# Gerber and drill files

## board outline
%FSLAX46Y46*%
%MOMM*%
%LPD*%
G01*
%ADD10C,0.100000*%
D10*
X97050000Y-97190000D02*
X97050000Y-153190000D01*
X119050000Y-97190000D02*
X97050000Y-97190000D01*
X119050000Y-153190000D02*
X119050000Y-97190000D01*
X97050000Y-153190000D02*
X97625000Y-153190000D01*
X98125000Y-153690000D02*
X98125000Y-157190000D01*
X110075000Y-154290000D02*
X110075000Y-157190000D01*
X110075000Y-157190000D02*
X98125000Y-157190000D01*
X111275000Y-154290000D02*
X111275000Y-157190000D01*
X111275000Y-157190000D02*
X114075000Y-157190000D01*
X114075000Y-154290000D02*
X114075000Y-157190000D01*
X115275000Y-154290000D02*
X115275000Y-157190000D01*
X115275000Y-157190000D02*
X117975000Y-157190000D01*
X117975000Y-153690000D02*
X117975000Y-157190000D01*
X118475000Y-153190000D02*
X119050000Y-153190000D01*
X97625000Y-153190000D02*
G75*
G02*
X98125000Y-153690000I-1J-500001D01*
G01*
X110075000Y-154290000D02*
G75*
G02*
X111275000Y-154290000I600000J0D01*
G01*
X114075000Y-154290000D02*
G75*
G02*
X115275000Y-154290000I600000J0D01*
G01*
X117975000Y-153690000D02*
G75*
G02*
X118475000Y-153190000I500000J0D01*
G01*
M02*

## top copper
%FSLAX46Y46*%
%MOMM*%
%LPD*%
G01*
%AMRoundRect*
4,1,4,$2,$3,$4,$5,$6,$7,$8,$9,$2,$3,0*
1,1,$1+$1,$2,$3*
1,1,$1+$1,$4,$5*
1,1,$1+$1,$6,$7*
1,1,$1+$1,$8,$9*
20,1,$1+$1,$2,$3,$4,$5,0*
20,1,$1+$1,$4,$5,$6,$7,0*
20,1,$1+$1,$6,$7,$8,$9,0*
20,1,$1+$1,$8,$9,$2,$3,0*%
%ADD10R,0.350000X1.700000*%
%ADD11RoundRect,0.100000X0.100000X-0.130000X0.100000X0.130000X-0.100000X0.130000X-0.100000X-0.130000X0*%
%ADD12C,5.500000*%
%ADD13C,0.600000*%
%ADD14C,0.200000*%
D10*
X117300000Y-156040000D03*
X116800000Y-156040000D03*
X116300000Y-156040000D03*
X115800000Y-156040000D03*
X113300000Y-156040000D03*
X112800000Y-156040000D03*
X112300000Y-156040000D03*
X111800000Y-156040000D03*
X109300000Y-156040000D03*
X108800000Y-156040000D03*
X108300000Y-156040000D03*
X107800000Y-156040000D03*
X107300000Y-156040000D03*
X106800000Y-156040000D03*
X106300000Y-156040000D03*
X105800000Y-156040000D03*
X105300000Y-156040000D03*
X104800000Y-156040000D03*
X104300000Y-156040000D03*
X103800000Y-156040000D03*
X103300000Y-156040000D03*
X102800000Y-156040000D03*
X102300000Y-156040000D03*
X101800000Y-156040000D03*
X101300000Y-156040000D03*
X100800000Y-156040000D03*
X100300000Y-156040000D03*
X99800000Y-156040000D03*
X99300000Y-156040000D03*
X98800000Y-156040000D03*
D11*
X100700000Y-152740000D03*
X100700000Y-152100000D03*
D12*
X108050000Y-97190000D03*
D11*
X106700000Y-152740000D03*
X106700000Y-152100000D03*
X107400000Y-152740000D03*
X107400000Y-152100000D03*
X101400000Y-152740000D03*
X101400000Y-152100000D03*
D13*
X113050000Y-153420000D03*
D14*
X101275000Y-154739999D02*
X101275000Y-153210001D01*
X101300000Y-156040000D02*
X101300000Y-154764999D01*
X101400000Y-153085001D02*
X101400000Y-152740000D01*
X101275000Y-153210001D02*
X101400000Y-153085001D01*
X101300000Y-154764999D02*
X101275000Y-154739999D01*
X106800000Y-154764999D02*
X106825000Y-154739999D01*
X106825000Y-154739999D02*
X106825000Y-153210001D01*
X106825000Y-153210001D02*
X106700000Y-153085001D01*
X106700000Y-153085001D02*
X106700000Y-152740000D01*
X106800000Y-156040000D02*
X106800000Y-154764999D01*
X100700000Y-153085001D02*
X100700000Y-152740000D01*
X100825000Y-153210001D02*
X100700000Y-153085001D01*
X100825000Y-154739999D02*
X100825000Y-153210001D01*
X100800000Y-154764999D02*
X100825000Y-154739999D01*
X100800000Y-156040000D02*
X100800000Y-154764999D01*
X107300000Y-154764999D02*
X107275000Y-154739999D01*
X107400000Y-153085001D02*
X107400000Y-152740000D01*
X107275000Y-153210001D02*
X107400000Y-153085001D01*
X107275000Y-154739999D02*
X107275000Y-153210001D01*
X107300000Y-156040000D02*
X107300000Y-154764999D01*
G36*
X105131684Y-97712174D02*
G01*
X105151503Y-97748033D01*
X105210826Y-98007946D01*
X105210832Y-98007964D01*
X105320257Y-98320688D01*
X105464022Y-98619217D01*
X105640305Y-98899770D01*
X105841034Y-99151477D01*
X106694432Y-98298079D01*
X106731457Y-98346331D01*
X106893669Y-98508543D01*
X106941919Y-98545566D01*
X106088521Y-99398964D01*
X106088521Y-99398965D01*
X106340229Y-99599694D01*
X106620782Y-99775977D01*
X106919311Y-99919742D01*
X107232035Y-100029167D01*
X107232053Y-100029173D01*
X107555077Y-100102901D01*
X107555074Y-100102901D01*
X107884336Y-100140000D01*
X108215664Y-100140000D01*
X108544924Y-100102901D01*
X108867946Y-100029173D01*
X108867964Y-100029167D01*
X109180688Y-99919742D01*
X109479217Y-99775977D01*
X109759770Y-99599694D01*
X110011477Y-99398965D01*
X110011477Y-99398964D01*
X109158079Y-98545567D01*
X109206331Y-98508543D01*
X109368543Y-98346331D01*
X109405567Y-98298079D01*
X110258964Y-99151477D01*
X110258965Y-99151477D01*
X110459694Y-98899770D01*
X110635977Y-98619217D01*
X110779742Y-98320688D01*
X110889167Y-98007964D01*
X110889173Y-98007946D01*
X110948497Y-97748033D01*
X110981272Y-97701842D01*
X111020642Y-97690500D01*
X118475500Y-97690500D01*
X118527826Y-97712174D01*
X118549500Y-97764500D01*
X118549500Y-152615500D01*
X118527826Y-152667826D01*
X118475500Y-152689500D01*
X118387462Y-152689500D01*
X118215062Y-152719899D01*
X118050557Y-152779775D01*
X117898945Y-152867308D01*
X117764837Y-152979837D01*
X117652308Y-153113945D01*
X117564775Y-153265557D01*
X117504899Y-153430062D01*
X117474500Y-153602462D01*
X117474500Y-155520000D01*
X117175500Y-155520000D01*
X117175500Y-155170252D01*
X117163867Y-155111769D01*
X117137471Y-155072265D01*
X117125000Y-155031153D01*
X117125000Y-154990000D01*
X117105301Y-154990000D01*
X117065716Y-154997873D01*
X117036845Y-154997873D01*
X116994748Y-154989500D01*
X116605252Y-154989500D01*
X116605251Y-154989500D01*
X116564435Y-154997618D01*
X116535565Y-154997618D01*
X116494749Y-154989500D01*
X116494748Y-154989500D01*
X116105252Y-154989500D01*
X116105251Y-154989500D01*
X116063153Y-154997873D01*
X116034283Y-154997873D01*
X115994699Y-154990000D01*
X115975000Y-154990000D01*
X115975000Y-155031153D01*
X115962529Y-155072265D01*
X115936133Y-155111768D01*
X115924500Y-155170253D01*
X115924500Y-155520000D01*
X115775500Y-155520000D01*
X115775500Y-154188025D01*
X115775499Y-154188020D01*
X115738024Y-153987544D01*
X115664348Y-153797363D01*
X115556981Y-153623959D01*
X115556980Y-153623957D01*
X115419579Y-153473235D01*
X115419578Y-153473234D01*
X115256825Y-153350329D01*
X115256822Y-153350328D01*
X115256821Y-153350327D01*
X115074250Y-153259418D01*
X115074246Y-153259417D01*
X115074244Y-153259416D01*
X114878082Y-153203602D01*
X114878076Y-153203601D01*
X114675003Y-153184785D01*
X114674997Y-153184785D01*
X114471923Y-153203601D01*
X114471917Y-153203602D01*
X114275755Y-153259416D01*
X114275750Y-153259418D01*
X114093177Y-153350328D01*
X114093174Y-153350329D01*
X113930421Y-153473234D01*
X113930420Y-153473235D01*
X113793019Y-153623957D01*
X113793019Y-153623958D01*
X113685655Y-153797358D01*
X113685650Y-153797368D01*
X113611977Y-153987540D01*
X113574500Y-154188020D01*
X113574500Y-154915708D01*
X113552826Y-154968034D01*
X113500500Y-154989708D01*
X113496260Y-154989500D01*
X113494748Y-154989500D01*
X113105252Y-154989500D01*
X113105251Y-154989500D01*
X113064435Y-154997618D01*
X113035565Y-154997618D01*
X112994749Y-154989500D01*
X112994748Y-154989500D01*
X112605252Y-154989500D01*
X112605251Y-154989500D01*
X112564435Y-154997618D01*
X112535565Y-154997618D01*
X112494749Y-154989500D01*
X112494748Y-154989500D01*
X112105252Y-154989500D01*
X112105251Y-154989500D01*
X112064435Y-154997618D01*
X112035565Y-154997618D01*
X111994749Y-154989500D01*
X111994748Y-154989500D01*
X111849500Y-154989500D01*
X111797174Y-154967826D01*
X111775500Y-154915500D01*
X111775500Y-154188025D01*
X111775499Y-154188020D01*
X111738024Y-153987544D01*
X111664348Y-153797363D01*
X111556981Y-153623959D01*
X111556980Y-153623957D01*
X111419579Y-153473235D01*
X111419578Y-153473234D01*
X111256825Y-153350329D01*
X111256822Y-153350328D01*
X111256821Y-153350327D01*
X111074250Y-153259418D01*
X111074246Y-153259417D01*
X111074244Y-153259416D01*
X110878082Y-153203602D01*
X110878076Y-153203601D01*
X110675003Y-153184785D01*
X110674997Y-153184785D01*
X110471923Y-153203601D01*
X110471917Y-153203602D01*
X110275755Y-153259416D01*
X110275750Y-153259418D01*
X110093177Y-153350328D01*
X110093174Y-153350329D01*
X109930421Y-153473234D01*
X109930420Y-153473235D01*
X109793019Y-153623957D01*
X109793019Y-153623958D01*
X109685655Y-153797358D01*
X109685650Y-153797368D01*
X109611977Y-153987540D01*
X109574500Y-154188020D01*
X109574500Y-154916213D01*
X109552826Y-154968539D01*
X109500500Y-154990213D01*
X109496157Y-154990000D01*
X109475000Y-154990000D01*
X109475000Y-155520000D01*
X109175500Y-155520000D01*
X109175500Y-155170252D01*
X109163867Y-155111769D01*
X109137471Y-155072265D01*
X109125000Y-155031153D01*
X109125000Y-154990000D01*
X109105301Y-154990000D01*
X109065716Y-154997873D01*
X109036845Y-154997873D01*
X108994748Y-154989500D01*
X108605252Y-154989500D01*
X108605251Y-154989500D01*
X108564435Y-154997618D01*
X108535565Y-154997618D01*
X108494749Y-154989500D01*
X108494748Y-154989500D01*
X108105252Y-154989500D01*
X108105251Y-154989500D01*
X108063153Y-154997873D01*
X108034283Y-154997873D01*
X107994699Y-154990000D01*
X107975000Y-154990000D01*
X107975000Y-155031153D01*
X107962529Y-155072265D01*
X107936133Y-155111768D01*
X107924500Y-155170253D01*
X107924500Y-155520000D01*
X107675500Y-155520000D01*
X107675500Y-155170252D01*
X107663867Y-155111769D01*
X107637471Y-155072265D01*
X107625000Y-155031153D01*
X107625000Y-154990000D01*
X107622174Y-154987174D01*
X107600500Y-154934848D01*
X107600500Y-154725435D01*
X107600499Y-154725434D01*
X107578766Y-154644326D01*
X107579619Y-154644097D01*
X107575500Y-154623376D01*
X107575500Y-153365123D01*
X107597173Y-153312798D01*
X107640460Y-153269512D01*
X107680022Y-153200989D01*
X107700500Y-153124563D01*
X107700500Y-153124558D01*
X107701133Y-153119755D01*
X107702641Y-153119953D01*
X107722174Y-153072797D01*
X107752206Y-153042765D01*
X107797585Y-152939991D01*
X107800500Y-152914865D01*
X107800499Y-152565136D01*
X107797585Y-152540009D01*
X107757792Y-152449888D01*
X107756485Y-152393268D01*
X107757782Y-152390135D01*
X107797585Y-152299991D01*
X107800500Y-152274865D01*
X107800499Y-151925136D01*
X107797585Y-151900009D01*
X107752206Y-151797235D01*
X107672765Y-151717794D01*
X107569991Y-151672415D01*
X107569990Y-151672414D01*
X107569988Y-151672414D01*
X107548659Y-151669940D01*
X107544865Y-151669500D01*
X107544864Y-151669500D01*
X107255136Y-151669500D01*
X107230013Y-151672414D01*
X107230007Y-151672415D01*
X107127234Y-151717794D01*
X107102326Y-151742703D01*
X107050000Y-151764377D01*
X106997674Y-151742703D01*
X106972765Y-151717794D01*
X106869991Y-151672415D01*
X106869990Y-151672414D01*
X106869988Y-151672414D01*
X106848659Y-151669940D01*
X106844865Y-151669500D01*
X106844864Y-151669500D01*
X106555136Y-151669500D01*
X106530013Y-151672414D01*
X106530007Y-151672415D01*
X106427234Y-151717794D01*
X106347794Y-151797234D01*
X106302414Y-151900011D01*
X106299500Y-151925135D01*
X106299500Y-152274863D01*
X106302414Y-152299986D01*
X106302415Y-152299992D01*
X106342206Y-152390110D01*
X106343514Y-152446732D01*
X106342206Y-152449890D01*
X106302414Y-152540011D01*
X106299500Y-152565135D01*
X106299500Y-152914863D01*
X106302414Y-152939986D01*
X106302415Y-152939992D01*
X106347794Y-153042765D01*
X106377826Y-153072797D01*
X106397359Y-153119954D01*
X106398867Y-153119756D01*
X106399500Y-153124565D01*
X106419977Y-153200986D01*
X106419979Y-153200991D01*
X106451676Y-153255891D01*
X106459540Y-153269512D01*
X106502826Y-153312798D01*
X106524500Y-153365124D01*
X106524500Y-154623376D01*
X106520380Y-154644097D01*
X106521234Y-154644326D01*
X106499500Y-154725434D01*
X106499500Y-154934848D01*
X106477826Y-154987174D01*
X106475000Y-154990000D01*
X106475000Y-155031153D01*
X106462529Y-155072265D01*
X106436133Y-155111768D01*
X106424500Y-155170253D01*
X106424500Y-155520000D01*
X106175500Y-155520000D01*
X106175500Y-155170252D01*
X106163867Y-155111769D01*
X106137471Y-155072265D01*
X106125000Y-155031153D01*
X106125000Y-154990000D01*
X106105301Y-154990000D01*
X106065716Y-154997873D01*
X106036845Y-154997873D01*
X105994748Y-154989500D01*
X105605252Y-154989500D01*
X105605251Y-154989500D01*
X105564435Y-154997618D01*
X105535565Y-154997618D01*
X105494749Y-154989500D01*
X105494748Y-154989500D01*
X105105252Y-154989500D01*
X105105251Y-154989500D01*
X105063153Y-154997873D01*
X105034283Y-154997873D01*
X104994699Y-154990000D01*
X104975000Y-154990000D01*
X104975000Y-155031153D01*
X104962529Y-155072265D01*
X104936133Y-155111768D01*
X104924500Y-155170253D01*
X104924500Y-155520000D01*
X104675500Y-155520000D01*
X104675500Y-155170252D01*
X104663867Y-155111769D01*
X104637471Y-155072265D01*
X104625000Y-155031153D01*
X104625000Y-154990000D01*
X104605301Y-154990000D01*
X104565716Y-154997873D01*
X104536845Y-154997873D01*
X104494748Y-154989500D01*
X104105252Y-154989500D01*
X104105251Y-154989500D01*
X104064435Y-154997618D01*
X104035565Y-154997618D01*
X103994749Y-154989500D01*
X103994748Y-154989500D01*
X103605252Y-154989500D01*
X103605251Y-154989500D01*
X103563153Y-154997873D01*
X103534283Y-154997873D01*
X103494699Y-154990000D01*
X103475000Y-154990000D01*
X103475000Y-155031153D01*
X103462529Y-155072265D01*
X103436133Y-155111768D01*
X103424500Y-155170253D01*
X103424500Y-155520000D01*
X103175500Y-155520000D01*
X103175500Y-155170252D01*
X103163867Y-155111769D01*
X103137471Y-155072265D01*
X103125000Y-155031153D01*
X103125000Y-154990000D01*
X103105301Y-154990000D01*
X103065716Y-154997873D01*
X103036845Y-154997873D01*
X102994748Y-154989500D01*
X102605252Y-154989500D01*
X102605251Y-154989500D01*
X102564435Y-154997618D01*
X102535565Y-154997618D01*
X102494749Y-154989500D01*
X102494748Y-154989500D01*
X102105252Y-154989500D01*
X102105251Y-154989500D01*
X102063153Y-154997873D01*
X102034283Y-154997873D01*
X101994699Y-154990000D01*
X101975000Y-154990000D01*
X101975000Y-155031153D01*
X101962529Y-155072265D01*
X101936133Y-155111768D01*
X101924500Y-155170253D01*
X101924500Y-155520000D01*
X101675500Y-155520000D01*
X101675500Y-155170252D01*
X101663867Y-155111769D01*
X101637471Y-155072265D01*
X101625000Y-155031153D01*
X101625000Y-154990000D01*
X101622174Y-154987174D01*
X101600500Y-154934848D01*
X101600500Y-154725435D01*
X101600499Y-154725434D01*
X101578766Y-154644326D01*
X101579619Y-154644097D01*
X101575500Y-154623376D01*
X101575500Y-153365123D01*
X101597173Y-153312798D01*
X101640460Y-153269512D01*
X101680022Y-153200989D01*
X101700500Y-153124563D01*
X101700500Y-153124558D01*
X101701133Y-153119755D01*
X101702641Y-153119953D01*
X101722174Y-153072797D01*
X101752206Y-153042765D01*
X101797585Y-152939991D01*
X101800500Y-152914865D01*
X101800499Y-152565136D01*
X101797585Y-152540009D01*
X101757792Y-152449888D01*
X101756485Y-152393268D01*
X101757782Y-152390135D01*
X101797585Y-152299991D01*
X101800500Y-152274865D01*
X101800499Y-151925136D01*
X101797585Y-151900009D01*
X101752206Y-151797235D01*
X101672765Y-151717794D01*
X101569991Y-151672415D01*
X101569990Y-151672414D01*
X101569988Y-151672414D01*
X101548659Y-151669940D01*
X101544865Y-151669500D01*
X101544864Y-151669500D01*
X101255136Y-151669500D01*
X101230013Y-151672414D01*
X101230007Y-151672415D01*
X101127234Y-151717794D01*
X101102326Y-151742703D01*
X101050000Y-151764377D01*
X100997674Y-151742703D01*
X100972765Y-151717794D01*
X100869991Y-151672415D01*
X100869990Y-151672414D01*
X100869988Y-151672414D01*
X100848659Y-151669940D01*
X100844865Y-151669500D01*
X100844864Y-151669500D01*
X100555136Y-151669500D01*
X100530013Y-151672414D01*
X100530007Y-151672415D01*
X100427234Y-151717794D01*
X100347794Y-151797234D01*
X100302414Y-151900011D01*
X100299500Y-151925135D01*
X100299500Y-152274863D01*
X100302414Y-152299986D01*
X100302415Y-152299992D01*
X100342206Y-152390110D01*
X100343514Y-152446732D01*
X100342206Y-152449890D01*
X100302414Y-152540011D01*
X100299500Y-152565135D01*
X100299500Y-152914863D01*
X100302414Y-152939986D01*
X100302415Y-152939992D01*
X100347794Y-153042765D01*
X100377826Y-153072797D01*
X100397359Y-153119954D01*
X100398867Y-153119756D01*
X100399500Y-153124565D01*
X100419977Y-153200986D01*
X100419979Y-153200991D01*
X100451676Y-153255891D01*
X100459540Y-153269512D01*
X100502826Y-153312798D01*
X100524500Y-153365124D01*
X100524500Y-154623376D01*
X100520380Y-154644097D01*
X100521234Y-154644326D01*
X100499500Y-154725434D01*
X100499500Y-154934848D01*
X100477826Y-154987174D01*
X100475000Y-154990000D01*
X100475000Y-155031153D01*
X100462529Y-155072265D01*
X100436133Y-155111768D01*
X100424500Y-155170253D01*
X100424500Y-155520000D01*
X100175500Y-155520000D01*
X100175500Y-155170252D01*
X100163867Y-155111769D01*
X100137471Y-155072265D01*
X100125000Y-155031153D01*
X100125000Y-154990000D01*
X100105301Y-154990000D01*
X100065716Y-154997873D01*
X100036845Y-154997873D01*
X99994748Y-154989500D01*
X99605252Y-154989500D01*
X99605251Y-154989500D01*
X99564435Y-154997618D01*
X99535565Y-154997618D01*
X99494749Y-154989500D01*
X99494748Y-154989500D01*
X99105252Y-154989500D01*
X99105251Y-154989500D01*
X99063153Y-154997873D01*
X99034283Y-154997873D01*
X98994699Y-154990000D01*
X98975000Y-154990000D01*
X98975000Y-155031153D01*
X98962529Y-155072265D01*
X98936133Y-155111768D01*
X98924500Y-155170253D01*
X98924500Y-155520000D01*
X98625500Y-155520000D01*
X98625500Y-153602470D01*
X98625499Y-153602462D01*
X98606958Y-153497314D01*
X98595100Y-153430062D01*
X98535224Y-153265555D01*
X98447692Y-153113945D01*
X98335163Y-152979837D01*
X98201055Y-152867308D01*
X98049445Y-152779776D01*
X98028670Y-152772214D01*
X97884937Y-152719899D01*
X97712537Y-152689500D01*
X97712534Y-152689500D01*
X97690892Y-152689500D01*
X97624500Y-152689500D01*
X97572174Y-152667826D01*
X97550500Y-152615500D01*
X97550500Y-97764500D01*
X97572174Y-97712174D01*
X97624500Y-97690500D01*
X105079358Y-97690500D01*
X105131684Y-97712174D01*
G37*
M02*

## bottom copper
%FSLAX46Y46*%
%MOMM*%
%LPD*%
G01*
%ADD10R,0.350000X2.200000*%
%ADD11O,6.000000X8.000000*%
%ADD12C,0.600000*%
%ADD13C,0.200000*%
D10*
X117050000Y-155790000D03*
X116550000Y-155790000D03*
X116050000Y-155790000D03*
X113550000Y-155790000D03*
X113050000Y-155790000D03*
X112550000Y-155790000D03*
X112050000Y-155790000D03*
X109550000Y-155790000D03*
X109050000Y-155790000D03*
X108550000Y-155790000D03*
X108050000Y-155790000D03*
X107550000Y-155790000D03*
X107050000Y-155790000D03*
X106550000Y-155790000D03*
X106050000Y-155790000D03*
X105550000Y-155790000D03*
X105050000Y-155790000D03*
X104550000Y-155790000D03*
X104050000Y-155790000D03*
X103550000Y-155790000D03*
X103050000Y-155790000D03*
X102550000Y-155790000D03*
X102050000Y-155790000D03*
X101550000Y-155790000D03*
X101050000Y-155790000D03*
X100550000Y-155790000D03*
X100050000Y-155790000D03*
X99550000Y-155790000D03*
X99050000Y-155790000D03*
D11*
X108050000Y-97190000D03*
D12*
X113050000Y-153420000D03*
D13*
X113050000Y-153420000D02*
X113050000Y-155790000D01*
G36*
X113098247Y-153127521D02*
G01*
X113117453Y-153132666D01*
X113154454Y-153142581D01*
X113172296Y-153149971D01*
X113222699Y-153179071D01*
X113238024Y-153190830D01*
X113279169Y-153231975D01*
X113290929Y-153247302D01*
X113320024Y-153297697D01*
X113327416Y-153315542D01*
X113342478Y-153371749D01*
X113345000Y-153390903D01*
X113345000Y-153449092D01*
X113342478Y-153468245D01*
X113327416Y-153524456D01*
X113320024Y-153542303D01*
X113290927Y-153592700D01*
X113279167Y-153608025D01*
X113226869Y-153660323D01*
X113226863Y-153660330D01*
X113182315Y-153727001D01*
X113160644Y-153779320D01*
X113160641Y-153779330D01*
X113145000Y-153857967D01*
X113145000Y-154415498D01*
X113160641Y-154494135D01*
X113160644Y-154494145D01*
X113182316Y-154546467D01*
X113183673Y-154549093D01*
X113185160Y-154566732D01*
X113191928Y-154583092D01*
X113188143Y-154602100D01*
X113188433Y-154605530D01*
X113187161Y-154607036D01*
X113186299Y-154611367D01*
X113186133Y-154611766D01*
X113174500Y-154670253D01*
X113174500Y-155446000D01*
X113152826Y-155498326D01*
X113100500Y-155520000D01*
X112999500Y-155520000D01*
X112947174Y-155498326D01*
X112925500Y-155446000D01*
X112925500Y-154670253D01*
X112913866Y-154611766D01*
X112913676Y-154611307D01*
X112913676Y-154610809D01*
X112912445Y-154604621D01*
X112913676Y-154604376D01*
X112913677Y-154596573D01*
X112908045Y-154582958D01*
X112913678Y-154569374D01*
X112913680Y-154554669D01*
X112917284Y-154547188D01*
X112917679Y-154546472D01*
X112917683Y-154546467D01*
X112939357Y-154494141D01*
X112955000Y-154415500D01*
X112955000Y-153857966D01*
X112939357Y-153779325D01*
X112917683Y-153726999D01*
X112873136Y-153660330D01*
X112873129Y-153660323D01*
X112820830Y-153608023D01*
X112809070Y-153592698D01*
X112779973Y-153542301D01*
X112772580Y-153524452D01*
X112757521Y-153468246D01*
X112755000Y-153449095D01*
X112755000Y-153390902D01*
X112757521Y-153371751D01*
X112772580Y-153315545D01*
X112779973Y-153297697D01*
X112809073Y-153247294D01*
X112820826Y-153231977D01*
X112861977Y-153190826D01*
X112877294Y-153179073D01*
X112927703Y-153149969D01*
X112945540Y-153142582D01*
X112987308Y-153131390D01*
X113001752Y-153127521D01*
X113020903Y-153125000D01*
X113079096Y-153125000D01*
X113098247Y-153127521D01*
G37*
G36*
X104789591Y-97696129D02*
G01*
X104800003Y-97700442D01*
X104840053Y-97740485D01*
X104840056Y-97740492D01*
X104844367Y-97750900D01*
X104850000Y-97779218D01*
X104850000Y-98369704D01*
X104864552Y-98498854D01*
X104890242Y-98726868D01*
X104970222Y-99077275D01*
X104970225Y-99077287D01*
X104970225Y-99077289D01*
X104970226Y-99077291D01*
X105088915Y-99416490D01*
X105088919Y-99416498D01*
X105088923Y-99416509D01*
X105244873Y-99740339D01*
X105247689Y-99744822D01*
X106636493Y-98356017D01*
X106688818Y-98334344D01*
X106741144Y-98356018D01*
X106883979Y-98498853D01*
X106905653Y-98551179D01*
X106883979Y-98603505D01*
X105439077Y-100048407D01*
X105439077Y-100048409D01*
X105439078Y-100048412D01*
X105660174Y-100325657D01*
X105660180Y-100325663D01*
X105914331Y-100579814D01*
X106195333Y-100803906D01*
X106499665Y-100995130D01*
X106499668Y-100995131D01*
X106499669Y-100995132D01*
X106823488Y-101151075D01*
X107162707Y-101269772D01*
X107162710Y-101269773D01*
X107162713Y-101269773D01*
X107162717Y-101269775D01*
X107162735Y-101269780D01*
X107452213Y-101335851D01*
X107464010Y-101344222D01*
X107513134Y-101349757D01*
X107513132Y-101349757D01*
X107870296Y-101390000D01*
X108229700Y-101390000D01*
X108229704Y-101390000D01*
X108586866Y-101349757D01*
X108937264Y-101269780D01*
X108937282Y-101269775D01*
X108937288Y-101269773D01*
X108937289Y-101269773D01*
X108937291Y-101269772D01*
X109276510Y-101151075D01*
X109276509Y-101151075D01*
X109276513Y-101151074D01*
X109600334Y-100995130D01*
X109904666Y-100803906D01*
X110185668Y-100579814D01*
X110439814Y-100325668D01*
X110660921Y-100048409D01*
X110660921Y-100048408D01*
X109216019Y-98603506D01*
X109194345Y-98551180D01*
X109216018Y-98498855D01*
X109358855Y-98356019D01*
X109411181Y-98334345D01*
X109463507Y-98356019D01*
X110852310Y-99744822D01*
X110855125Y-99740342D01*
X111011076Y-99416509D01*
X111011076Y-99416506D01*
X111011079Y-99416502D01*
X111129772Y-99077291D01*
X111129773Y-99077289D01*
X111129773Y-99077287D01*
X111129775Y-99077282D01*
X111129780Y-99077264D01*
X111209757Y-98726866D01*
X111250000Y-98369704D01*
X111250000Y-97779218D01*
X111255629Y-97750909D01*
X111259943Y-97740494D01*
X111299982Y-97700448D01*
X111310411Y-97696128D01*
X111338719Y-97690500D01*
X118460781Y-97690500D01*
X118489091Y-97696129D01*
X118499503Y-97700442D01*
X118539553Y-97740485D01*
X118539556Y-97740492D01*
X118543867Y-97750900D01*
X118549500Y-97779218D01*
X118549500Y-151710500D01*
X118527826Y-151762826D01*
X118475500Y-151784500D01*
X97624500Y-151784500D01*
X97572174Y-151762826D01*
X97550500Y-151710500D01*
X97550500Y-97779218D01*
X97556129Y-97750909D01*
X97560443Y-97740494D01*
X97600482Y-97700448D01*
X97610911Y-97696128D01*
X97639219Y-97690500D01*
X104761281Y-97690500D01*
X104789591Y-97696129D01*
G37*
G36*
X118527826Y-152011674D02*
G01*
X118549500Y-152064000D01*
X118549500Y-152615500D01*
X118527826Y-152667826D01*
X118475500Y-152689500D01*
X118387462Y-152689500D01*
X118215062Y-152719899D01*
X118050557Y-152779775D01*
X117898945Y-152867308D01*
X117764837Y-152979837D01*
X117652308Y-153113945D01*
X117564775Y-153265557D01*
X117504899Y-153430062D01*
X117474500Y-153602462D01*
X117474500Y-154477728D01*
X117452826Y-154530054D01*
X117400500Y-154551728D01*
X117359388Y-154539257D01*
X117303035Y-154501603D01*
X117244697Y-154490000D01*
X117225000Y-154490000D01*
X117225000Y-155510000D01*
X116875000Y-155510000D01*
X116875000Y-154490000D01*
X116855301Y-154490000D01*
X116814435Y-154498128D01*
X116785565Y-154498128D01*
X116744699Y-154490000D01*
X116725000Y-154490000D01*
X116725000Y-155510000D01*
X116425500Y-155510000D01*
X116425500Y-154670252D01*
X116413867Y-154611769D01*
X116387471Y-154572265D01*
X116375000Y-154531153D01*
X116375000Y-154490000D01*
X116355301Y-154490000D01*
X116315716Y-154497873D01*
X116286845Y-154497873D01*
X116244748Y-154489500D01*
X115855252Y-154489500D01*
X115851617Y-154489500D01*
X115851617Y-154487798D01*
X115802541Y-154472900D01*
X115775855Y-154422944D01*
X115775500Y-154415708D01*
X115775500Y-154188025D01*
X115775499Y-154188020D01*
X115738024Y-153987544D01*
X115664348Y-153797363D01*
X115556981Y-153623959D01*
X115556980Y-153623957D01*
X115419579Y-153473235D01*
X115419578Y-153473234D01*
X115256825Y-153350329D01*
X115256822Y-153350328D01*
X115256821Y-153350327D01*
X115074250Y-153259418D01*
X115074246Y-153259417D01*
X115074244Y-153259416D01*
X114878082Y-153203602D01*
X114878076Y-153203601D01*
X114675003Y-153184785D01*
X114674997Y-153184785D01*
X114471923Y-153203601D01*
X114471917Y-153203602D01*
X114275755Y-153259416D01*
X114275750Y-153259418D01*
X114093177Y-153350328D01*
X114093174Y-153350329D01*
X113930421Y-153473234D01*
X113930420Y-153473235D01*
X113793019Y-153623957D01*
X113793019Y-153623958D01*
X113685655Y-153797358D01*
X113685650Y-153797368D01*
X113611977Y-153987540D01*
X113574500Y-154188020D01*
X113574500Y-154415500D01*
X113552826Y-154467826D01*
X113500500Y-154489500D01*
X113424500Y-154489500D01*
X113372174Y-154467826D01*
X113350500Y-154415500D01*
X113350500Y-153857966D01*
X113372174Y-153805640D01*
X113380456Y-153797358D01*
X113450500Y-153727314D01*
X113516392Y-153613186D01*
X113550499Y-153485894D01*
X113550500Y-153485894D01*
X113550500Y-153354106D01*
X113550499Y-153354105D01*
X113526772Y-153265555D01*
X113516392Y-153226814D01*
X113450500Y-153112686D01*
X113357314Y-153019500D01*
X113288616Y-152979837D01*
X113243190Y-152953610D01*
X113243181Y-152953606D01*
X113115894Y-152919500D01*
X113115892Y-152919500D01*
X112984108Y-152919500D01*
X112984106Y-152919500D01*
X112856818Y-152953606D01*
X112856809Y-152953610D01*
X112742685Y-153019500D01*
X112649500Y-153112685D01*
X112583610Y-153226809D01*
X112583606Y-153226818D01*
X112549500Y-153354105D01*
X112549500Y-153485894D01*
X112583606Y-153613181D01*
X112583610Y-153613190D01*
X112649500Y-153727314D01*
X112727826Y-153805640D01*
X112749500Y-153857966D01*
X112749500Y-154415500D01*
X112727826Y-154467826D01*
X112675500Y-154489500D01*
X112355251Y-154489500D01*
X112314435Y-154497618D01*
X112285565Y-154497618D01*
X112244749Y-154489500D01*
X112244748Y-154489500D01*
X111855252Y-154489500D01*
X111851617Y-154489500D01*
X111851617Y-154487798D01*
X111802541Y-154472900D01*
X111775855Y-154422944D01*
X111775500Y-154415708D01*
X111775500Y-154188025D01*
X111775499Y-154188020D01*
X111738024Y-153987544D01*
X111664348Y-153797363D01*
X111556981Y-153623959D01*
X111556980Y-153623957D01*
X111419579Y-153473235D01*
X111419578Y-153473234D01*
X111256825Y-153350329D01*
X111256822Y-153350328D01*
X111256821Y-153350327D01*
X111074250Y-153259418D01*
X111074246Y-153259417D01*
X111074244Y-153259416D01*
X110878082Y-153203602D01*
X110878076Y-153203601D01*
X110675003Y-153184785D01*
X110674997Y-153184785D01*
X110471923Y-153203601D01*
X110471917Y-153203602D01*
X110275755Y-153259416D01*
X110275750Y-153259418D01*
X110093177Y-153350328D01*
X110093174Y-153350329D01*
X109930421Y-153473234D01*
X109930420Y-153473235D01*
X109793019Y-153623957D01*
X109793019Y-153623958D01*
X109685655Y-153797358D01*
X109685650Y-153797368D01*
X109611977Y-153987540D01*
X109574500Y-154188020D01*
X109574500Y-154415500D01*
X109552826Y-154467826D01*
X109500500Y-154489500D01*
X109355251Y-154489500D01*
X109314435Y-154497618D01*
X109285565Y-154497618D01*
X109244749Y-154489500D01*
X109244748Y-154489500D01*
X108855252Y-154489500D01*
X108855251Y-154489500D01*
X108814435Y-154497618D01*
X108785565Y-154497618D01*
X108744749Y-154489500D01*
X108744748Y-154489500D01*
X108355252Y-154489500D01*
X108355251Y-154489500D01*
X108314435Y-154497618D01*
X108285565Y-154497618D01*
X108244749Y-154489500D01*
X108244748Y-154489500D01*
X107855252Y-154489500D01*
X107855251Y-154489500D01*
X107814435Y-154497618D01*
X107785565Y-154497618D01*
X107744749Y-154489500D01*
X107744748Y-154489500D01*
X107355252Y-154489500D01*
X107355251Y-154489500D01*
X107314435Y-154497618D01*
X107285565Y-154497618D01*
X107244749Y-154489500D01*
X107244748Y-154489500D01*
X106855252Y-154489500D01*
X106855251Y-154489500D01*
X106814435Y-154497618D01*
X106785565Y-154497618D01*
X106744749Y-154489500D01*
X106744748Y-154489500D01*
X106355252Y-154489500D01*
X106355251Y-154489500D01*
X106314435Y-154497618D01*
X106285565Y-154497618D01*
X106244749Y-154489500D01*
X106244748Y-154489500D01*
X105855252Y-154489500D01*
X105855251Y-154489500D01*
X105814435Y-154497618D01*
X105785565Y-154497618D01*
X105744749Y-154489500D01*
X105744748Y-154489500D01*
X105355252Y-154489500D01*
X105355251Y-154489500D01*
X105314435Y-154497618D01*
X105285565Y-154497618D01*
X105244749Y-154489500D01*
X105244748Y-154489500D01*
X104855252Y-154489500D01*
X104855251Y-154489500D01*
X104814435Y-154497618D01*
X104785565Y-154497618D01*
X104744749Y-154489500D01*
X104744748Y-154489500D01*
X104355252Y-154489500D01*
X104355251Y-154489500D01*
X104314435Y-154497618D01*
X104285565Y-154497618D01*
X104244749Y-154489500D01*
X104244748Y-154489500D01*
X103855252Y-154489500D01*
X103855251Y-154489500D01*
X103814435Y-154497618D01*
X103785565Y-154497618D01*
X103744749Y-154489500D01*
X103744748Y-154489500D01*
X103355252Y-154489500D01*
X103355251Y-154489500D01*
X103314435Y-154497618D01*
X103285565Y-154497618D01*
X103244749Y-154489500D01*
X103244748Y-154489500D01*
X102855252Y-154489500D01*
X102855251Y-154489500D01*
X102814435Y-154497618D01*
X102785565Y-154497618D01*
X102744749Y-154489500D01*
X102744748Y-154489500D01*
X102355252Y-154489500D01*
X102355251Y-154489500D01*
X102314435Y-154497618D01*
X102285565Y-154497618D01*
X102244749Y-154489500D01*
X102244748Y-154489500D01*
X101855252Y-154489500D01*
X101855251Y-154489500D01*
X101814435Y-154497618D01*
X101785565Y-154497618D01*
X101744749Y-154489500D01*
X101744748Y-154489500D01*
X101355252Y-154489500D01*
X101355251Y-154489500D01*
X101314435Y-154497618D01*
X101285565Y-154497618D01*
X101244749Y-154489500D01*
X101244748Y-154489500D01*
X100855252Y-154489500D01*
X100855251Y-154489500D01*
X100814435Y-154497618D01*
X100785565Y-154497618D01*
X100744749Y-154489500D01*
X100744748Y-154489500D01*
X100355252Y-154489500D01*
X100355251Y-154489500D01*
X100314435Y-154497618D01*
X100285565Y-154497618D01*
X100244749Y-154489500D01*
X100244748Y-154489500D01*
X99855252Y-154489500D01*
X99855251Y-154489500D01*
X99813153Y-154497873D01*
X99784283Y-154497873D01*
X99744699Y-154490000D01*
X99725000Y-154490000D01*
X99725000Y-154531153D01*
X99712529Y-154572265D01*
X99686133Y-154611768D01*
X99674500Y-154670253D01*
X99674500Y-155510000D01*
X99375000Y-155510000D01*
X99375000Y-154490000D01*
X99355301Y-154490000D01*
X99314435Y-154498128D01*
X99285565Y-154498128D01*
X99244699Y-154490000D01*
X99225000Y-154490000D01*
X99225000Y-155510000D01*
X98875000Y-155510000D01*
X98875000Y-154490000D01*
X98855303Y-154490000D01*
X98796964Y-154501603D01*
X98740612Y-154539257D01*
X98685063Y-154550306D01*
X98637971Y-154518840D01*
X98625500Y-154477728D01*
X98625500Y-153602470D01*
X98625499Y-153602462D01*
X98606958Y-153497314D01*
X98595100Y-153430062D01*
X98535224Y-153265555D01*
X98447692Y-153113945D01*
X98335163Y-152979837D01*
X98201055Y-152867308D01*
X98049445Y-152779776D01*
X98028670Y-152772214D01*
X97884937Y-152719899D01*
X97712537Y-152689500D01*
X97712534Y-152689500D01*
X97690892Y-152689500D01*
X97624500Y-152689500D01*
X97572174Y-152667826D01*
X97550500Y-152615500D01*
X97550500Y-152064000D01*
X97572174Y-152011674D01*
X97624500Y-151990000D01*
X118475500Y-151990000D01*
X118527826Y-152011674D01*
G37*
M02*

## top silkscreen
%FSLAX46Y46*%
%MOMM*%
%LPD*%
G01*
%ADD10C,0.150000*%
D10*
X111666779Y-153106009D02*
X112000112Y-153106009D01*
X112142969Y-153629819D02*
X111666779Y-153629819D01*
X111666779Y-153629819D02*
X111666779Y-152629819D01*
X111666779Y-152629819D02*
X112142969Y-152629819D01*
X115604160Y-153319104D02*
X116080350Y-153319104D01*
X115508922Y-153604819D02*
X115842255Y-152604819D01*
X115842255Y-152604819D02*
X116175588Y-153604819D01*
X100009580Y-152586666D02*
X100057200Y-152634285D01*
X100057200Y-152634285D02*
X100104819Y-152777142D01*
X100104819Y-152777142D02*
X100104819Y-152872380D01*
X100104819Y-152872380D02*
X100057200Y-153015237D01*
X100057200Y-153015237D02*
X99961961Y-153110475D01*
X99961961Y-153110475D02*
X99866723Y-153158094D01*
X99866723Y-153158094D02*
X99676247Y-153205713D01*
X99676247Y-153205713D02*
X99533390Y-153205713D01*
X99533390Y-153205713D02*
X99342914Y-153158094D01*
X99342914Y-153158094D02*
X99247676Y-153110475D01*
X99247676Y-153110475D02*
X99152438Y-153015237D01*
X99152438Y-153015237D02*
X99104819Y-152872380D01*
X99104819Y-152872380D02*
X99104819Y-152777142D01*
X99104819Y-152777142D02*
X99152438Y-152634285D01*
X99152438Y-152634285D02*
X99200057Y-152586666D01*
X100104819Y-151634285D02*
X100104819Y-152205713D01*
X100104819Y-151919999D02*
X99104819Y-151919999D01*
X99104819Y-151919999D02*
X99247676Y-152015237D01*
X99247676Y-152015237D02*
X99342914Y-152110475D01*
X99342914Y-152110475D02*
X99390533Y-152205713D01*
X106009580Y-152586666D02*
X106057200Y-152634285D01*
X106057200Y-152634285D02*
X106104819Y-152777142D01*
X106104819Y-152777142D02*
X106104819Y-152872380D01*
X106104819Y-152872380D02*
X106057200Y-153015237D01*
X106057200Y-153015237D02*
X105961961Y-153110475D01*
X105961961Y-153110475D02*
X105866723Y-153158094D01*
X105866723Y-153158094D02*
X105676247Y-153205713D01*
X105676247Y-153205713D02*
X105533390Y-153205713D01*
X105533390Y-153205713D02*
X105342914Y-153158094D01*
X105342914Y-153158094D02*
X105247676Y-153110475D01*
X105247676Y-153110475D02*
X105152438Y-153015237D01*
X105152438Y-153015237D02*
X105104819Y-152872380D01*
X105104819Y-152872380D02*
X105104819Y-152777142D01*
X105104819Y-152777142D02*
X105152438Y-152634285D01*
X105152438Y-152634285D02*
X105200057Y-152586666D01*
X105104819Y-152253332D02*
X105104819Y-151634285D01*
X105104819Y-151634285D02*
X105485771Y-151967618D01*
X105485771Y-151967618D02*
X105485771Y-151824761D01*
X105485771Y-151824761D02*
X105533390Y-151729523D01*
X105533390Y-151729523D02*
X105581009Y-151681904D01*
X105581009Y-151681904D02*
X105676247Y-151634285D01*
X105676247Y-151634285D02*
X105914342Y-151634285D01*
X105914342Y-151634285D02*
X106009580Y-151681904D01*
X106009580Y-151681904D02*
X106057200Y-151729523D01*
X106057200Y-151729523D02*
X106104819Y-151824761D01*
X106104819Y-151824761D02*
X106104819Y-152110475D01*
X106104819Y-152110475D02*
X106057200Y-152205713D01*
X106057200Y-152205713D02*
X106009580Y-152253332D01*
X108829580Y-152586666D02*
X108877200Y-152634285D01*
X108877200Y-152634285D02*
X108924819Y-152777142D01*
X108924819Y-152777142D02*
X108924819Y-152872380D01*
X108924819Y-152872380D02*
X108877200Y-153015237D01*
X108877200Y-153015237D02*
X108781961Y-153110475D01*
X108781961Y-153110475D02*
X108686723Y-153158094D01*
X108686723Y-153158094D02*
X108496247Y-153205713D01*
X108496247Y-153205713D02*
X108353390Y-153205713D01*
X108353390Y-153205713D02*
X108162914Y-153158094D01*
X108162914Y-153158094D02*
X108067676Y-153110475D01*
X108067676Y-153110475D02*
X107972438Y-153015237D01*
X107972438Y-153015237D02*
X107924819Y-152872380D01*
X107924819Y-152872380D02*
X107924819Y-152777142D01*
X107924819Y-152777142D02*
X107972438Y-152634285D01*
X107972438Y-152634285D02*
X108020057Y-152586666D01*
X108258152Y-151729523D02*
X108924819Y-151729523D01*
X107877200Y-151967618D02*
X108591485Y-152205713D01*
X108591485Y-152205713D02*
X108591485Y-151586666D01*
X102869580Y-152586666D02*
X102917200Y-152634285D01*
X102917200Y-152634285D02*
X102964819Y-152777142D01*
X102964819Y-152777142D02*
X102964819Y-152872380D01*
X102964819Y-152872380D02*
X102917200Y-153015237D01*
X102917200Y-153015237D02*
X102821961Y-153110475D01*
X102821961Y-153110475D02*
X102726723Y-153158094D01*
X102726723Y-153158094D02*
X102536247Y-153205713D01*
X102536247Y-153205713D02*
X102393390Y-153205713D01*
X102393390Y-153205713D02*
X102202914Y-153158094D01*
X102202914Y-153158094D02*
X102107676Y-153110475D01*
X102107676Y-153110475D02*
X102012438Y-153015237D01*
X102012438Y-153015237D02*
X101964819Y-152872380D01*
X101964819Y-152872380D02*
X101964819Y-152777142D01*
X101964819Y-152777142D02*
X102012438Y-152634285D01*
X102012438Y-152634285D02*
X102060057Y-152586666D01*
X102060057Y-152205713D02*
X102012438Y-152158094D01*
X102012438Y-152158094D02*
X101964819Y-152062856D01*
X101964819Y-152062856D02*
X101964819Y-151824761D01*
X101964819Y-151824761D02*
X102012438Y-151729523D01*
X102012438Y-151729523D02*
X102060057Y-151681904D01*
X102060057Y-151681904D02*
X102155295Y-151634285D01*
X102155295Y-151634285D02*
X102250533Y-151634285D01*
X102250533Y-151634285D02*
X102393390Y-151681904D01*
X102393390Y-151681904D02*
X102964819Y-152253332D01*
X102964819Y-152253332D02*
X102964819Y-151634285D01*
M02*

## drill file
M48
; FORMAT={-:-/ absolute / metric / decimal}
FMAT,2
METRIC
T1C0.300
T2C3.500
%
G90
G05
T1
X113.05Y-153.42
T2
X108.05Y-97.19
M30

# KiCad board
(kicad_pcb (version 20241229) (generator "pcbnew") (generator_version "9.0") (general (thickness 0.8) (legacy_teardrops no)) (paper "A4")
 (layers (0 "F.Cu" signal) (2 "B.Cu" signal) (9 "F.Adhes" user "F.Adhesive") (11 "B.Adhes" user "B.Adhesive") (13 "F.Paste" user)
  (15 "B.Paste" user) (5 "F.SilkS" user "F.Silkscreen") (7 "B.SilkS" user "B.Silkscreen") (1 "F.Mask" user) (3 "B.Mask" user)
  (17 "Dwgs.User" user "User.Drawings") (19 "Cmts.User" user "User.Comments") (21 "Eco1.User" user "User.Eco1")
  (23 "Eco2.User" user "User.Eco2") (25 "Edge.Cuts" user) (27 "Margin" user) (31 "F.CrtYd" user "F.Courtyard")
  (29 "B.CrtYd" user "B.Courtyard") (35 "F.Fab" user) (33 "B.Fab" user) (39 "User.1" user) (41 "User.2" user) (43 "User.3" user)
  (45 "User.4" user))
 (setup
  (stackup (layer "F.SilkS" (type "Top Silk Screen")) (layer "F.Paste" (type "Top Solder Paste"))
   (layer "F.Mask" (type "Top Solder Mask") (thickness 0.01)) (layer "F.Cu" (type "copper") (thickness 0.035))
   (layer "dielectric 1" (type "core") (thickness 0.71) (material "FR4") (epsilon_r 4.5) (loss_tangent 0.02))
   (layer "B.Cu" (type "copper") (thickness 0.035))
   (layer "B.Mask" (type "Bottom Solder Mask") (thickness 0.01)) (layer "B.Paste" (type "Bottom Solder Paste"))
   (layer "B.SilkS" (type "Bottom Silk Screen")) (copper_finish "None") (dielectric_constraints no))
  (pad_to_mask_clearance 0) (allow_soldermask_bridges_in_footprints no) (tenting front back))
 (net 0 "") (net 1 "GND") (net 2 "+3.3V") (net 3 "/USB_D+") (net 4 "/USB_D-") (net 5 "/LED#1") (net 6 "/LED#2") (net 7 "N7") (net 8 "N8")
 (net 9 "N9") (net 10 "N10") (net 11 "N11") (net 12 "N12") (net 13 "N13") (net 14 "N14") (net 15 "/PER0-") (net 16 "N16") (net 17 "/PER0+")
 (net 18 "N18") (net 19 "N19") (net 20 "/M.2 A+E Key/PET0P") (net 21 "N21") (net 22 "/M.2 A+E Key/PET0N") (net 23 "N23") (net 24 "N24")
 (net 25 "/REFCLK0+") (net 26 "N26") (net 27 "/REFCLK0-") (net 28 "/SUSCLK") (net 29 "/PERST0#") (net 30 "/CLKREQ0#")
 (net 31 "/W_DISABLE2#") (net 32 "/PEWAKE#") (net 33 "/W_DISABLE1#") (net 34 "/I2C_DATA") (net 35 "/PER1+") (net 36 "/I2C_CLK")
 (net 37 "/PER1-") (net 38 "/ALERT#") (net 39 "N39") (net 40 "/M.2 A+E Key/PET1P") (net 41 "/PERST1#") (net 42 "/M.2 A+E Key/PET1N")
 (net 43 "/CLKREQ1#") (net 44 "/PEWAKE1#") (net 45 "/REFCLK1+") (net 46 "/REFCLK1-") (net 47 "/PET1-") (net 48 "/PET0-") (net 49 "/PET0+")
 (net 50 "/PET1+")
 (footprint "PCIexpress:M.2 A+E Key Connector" (layer "F.Cu") (at 108.05 156.08)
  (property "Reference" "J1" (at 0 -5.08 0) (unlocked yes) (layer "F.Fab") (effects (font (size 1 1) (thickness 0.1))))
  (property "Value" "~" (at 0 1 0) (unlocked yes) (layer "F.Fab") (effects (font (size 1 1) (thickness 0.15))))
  (fp_line (start -11 -2.89) (end -10.425 -2.89) (stroke (width 0.1) (type default)) (layer "Edge.Cuts"))
  (fp_line (start -9.925 -2.39) (end -9.925 1.11) (stroke (width 0.1) (type default)) (layer "Edge.Cuts"))
  (fp_line (start 2.025 -1.79) (end 2.025 1.11) (stroke (width 0.1) (type default)) (layer "Edge.Cuts"))
  (fp_line (start 2.025 1.11) (end -9.925 1.11) (stroke (width 0.1) (type default)) (layer "Edge.Cuts"))
  (fp_line (start 3.225 -1.79) (end 3.225 1.11) (stroke (width 0.1) (type default)) (layer "Edge.Cuts"))
  (fp_line (start 3.225 1.11) (end 6.025 1.11) (stroke (width 0.1) (type default)) (layer "Edge.Cuts"))
  (fp_line (start 6.025 -1.79) (end 6.025 1.11) (stroke (width 0.1) (type default)) (layer "Edge.Cuts"))
  (fp_line (start 7.225 -1.79) (end 7.225 1.11) (stroke (width 0.1) (type default)) (layer "Edge.Cuts"))
  (fp_line (start 7.225 1.11) (end 9.925 1.11) (stroke (width 0.1) (type default)) (layer "Edge.Cuts"))
  (fp_line (start 9.925 -2.39) (end 9.925 1.11) (stroke (width 0.1) (type default)) (layer "Edge.Cuts"))
  (fp_line (start 10.425 -2.89) (end 11 -2.89) (stroke (width 0.1) (type default)) (layer "Edge.Cuts"))
  (fp_arc (start -10.425 -2.89) (mid -10.071447 -2.743553) (end -9.925 -2.39) (stroke (width 0.1) (type default)) (layer "Edge.Cuts"))
  (fp_arc (start 2.025 -1.79) (mid 2.625 -2.39) (end 3.225 -1.79) (stroke (width 0.1) (type default)) (layer "Edge.Cuts"))
  (fp_arc (start 6.025 -1.79) (mid 6.625 -2.39) (end 7.225 -1.79) (stroke (width 0.1) (type default)) (layer "Edge.Cuts"))
  (fp_arc (start 9.925 -2.39) (mid 10.071447 -2.743553) (end 10.425 -2.89) (stroke (width 0.1) (type default)) (layer "Edge.Cuts"))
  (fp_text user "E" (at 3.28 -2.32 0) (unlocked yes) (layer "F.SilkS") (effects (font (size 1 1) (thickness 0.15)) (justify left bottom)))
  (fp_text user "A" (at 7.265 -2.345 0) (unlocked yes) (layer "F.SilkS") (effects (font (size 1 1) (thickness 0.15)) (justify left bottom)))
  (pad "1" smd rect (at 9.25 -0.04 180) (size 0.35 1.7) (layers "F.Cu") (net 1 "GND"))
  (pad "2" smd rect (at 9 -0.29 180) (size 0.35 2.2) (layers "B.Cu") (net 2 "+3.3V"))
  (pad "3" smd rect (at 8.75 -0.04 180) (size 0.35 1.7) (layers "F.Cu") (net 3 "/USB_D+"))
  (pad "4" smd rect (at 8.5 -0.29 180) (size 0.35 2.2) (layers "B.Cu") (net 2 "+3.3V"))
  (pad "5" smd rect (at 8.25 -0.04 180) (size 0.35 1.7) (layers "F.Cu") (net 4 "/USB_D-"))
  (pad "6" smd rect (at 8 -0.29 180) (size 0.35 2.2) (layers "B.Cu") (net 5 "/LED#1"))
  (pad "7" smd rect (at 7.75 -0.04 180) (size 0.35 1.7) (layers "F.Cu") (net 1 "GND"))
  (pad "16" smd rect (at 5.5 -0.29 180) (size 0.35 2.2) (layers "B.Cu") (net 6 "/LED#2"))
  (pad "17" smd rect (at 5.25 -0.04 180) (size 0.35 1.7) (layers "F.Cu") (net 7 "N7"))
  (pad "18" smd rect (at 5 -0.29 180) (size 0.35 2.2) (layers "B.Cu") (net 1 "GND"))
  (pad "19" smd rect (at 4.75 -0.04 180) (size 0.35 1.7) (layers "F.Cu") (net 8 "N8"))
  (pad "20" smd rect (at 4.5 -0.29 180) (size 0.35 2.2) (layers "B.Cu") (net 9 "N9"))
  (pad "21" smd rect (at 4.25 -0.04 180) (size 0.35 1.7) (layers "F.Cu") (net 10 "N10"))
  (pad "22" smd rect (at 4 -0.29 180) (size 0.35 2.2) (layers "B.Cu") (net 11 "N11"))
  (pad "23" smd rect (at 3.75 -0.04 180) (size 0.35 1.7) (layers "F.Cu") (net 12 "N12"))
  (pad "32" smd rect (at 1.5 -0.29 180) (size 0.35 2.2) (layers "B.Cu") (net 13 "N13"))
  (pad "33" smd rect (at 1.25 -0.04 180) (size 0.35 1.7) (layers "F.Cu") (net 1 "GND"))
  (pad "34" smd rect (at 1 -0.29 180) (size 0.35 2.2) (layers "B.Cu") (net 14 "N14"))
  (pad "35" smd rect (at 0.75 -0.04 180) (size 0.35 1.7) (layers "F.Cu") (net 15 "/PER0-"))
  (pad "36" smd rect (at 0.5 -0.29 180) (size 0.35 2.2) (layers "B.Cu") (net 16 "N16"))
  (pad "37" smd rect (at 0.25 -0.04 180) (size 0.35 1.7) (layers "F.Cu") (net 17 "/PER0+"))
  (pad "38" smd rect (at 0 -0.29 180) (size 0.35 2.2) (layers "B.Cu") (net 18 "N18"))
  (pad "39" smd rect (at -0.25 -0.04 180) (size 0.35 1.7) (layers "F.Cu") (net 1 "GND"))
  (pad "40" smd rect (at -0.5 -0.29 180) (size 0.35 2.2) (layers "B.Cu") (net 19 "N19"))
  (pad "41" smd rect (at -0.75 -0.04 180) (size 0.35 1.7) (layers "F.Cu") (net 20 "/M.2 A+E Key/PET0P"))
  (pad "42" smd rect (at -1 -0.29 180) (size 0.35 2.2) (layers "B.Cu") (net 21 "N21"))
  (pad "43" smd rect (at -1.25 -0.04 180) (size 0.35 1.7) (layers "F.Cu") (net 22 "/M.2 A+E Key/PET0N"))
  (pad "44" smd rect (at -1.5 -0.29 180) (size 0.35 2.2) (layers "B.Cu") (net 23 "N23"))
  (pad "45" smd rect (at -1.75 -0.04 180) (size 0.35 1.7) (layers "F.Cu") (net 1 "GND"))
  (pad "46" smd rect (at -2 -0.29 180) (size 0.35 2.2) (layers "B.Cu") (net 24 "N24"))
  (pad "47" smd rect (at -2.25 -0.04 180) (size 0.35 1.7) (layers "F.Cu") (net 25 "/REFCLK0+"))
  (pad "48" smd rect (at -2.5 -0.29 180) (size 0.35 2.2) (layers "B.Cu") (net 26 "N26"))
  (pad "49" smd rect (at -2.75 -0.04 180) (size 0.35 1.7) (layers "F.Cu") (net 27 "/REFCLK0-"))
  (pad "50" smd rect (at -3 -0.29 180) (size 0.35 2.2) (layers "B.Cu") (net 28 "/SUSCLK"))
  (pad "51" smd rect (at -3.25 -0.04 180) (size 0.35 1.7) (layers "F.Cu") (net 1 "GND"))
  (pad "52" smd rect (at -3.5 -0.29 180) (size 0.35 2.2) (layers "B.Cu") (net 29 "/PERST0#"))
  (pad "53" smd rect (at -3.75 -0.04 180) (size 0.35 1.7) (layers "F.Cu") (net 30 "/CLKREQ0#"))
  (pad "54" smd rect (at -4 -0.29 180) (size 0.35 2.2) (layers "B.Cu") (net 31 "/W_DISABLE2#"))
  (pad "55" smd rect (at -4.25 -0.04 180) (size 0.35 1.7) (layers "F.Cu") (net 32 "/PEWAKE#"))
  (pad "56" smd rect (at -4.5 -0.29 180) (size 0.35 2.2) (layers "B.Cu") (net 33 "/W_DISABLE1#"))
  (pad "57" smd rect (at -4.75 -0.04 180) (size 0.35 1.7) (layers "F.Cu") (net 1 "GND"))
  (pad "58" smd rect (at -5 -0.29 180) (size 0.35 2.2) (layers "B.Cu") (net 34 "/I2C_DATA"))
  (pad "59" smd rect (at -5.25 -0.04 180) (size 0.35 1.7) (layers "F.Cu") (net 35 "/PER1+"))
  (pad "60" smd rect (at -5.5 -0.29 180) (size 0.35 2.2) (layers "B.Cu") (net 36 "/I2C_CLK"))
  (pad "61" smd rect (at -5.75 -0.04 180) (size 0.35 1.7) (layers "F.Cu") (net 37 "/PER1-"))
  (pad "62" smd rect (at -6 -0.29 180) (size 0.35 2.2) (layers "B.Cu") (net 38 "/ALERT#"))
  (pad "63" smd rect (at -6.25 -0.04 180) (size 0.35 1.7) (layers "F.Cu") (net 1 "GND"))
  (pad "64" smd rect (at -6.5 -0.29 180) (size 0.35 2.2) (layers "B.Cu") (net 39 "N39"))
  (pad "65" smd rect (at -6.75 -0.04 180) (size 0.35 1.7) (layers "F.Cu") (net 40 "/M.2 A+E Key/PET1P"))
  (pad "66" smd rect (at -7 -0.29 180) (size 0.35 2.2) (layers "B.Cu") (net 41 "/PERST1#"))
  (pad "67" smd rect (at -7.25 -0.04 180) (size 0.35 1.7) (layers "F.Cu") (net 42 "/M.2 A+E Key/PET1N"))
  (pad "68" smd rect (at -7.5 -0.29 180) (size 0.35 2.2) (layers "B.Cu") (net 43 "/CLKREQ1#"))
  (pad "69" smd rect (at -7.75 -0.04 180) (size 0.35 1.7) (layers "F.Cu") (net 1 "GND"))
  (pad "70" smd rect (at -8 -0.29 180) (size 0.35 2.2) (layers "B.Cu") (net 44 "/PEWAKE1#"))
  (pad "71" smd rect (at -8.25 -0.04 180) (size 0.35 1.7) (layers "F.Cu") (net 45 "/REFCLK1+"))
  (pad "72" smd rect (at -8.5 -0.29 180) (size 0.35 2.2) (layers "B.Cu") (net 2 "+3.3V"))
  (pad "73" smd rect (at -8.75 -0.04 180) (size 0.35 1.7) (layers "F.Cu") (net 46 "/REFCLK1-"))
  (pad "74" smd rect (at -9 -0.29 180) (size 0.35 2.2) (layers "B.Cu") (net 2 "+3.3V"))
  (pad "75" smd rect (at -9.25 -0.04 180) (size 0.35 1.7) (layers "F.Cu") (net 1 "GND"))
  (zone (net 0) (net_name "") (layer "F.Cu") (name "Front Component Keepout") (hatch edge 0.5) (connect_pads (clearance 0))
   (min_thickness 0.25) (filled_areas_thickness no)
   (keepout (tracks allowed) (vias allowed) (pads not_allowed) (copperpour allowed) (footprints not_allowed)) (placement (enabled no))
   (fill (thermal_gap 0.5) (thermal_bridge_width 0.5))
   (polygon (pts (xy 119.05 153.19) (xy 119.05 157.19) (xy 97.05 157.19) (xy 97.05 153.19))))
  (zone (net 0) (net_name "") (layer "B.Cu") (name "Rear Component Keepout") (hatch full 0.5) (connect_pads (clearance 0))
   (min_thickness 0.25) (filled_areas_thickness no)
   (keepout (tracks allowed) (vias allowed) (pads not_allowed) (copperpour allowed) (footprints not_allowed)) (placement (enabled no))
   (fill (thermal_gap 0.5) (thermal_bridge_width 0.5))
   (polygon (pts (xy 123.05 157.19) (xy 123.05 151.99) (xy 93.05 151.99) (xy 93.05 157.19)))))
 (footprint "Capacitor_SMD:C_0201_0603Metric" (layer "F.Cu") (at 100.7 152.42 90)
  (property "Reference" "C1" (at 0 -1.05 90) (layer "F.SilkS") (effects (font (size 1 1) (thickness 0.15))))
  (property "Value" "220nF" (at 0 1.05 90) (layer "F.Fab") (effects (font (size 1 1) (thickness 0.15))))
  (pad "" smd roundrect (at -0.345 0 90) (size 0.318 0.36) (layers "F.Paste") (roundrect_rratio 0.25))
  (pad "" smd roundrect (at 0.345 0 90) (size 0.318 0.36) (layers "F.Paste") (roundrect_rratio 0.25))
  (pad "1" smd roundrect (at -0.32 0 90) (size 0.46 0.4) (layers "F.Cu" "F.Mask") (roundrect_rratio 0.25) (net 42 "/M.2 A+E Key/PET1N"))
  (pad "2" smd roundrect (at 0.32 0 90) (size 0.46 0.4) (layers "F.Cu" "F.Mask") (roundrect_rratio 0.25) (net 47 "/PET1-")))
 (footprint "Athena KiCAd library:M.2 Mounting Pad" (layer "F.Cu") (at 108.05 97.19)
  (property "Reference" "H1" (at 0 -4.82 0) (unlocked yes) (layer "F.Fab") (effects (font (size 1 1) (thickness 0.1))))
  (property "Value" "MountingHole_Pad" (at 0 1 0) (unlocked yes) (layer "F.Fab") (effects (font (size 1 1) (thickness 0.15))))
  (pad "1" thru_hole circle (at 0 0) (size 5.5 5.5) (drill 3.5) (layers "*.Cu" "*.Mask") (remove_unused_layers no) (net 1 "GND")
   (padstack (mode front_inner_back)
    (layer "Inner" (shape circle) (size 5.5 5.5) (zone_connect -1))
    (layer "B.Cu" (shape oval) (size 6 8) (thermal_bridge_angle 45) (zone_connect -1)))))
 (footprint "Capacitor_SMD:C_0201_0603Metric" (layer "F.Cu") (at 106.7 152.42 90)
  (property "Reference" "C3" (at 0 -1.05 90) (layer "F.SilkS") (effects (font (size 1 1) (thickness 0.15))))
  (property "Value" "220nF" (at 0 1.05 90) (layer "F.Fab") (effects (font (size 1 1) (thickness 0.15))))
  (pad "" smd roundrect (at -0.345 0 90) (size 0.318 0.36) (layers "F.Paste") (roundrect_rratio 0.25))
  (pad "" smd roundrect (at 0.345 0 90) (size 0.318 0.36) (layers "F.Paste") (roundrect_rratio 0.25))
  (pad "1" smd roundrect (at -0.32 0 90) (size 0.46 0.4) (layers "F.Cu" "F.Mask") (roundrect_rratio 0.25) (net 22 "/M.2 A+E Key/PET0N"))
  (pad "2" smd roundrect (at 0.32 0 90) (size 0.46 0.4) (layers "F.Cu" "F.Mask") (roundrect_rratio 0.25) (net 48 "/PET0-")))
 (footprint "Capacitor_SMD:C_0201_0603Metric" (layer "F.Cu") (at 107.4 152.42 90)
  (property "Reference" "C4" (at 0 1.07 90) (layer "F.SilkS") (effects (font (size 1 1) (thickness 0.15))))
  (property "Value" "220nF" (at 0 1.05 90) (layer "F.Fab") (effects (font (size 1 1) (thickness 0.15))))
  (pad "" smd roundrect (at -0.345 0 90) (size 0.318 0.36) (layers "F.Paste") (roundrect_rratio 0.25))
  (pad "" smd roundrect (at 0.345 0 90) (size 0.318 0.36) (layers "F.Paste") (roundrect_rratio 0.25))
  (pad "1" smd roundrect (at -0.32 0 90) (size 0.46 0.4) (layers "F.Cu" "F.Mask") (roundrect_rratio 0.25) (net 20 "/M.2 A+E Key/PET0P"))
  (pad "2" smd roundrect (at 0.32 0 90) (size 0.46 0.4) (layers "F.Cu" "F.Mask") (roundrect_rratio 0.25) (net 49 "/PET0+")))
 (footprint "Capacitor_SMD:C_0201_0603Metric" (layer "F.Cu") (at 101.4 152.42 90)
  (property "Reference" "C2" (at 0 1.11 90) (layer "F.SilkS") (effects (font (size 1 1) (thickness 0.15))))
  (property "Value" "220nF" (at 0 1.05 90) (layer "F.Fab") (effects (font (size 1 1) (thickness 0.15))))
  (pad "" smd roundrect (at -0.345 0 90) (size 0.318 0.36) (layers "F.Paste") (roundrect_rratio 0.25))
  (pad "" smd roundrect (at 0.345 0 90) (size 0.318 0.36) (layers "F.Paste") (roundrect_rratio 0.25))
  (pad "1" smd roundrect (at -0.32 0 90) (size 0.46 0.4) (layers "F.Cu" "F.Mask") (roundrect_rratio 0.25) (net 40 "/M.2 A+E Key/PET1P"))
  (pad "2" smd roundrect (at 0.32 0 90) (size 0.46 0.4) (layers "F.Cu" "F.Mask") (roundrect_rratio 0.25) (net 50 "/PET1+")))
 (gr_line (start 97.05 97.19) (end 97.05 153.19) (stroke (width 0.1) (type default)) (layer "Edge.Cuts"))
 (gr_line (start 119.05 97.19) (end 97.05 97.19) (stroke (width 0.1) (type default)) (layer "Edge.Cuts"))
 (gr_line (start 119.05 153.19) (end 119.05 97.19) (stroke (width 0.1) (type default)) (layer "Edge.Cuts"))
 (via (at 113.05 153.42) (size 0.6) (drill 0.3) (layers "F.Cu" "B.Cu") (free yes) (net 1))
 (segment (start 113.05 153.42) (end 113.05 155.79) (width 0.2) (layer "B.Cu") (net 1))
 (segment (start 101.275 154.739999) (end 101.275 153.210001) (width 0.2) (layer "F.Cu") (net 40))
 (segment (start 101.3 156.04) (end 101.3 154.764999) (width 0.2) (layer "F.Cu") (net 40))
 (segment (start 101.4 153.085001) (end 101.4 152.74) (width 0.2) (layer "F.Cu") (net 40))
 (segment (start 101.275 153.210001) (end 101.4 153.085001) (width 0.2) (layer "F.Cu") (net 40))
 (segment (start 101.3 154.764999) (end 101.275 154.739999) (width 0.2) (layer "F.Cu") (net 40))
 (segment (start 106.8 154.764999) (end 106.825 154.739999) (width 0.2) (layer "F.Cu") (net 22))
 (segment (start 106.825 154.739999) (end 106.825 153.210001) (width 0.2) (layer "F.Cu") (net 22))
 (segment (start 106.825 153.210001) (end 106.7 153.085001) (width 0.2) (layer "F.Cu") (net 22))
 (segment (start 106.7 153.085001) (end 106.7 152.74) (width 0.2) (layer "F.Cu") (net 22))
 (segment (start 106.8 156.04) (end 106.8 154.764999) (width 0.2) (layer "F.Cu") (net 22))
 (segment (start 100.7 153.085001) (end 100.7 152.74) (width 0.2) (layer "F.Cu") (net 42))
 (segment (start 100.825 153.210001) (end 100.7 153.085001) (width 0.2) (layer "F.Cu") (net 42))
 (segment (start 100.825 154.739999) (end 100.825 153.210001) (width 0.2) (layer "F.Cu") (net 42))
 (segment (start 100.8 154.764999) (end 100.825 154.739999) (width 0.2) (layer "F.Cu") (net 42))
 (segment (start 100.8 156.04) (end 100.8 154.764999) (width 0.2) (layer "F.Cu") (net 42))
 (segment (start 107.3 154.764999) (end 107.275 154.739999) (width 0.2) (layer "F.Cu") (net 20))
 (segment (start 107.4 153.085001) (end 107.4 152.74) (width 0.2) (layer "F.Cu") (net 20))
 (segment (start 107.275 153.210001) (end 107.4 153.085001) (width 0.2) (layer "F.Cu") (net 20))
 (segment (start 107.275 154.739999) (end 107.275 153.210001) (width 0.2) (layer "F.Cu") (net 20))
 (segment (start 107.3 156.04) (end 107.3 154.764999) (width 0.2) (layer "F.Cu") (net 20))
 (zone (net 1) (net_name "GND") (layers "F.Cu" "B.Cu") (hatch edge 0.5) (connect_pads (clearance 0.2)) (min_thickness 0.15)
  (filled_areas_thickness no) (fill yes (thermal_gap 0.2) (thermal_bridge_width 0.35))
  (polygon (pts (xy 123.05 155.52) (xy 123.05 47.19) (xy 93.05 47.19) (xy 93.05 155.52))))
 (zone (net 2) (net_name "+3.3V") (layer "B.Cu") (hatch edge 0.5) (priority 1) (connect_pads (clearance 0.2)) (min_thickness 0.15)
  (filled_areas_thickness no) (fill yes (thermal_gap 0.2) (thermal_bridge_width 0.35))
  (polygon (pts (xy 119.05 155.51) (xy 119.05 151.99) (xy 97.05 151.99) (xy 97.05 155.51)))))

